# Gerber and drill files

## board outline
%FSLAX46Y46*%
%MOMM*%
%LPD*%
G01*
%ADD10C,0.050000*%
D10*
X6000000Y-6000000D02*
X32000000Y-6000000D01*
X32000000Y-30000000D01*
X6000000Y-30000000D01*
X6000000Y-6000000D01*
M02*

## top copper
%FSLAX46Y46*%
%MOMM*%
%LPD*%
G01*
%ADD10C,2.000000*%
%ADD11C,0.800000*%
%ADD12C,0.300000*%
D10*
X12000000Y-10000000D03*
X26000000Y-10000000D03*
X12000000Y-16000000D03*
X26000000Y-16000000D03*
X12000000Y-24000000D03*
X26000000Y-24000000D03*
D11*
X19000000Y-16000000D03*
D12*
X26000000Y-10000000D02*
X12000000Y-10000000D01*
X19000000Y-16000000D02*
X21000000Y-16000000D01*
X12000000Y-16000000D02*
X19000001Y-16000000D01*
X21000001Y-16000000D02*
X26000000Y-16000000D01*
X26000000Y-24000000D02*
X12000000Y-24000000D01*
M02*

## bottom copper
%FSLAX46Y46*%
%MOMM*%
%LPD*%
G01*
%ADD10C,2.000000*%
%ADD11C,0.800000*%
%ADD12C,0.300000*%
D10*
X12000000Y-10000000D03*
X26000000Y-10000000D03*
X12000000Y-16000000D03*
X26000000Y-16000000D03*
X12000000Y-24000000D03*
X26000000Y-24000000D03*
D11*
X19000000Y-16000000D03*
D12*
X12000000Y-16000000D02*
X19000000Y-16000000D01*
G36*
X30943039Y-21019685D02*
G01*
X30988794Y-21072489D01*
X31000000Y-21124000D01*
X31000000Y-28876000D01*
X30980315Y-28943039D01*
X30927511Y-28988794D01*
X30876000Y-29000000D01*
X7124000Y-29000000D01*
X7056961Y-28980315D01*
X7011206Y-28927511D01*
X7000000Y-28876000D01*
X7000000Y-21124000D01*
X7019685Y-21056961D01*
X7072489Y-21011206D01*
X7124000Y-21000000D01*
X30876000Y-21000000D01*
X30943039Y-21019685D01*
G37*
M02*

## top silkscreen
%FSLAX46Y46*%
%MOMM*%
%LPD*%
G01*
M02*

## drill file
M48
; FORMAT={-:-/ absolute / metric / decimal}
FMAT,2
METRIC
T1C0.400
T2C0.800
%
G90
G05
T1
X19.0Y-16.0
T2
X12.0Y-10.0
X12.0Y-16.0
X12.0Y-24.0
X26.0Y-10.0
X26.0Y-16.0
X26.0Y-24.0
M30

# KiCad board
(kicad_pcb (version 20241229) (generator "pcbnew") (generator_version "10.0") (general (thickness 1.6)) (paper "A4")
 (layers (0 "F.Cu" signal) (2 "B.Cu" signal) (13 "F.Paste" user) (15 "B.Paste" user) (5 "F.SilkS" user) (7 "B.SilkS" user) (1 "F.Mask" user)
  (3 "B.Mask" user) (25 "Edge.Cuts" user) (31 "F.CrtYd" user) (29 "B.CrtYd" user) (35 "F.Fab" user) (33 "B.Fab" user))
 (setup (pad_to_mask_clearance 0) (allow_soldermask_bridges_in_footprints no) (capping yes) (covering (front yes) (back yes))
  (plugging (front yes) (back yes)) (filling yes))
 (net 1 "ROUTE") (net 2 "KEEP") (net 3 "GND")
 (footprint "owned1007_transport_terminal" (layer "F.Cu") (at 12 10)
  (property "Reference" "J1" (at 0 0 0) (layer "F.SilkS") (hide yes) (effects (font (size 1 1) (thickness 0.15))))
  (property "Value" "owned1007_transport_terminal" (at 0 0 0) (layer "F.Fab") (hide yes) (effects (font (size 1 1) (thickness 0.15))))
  (pad "1" thru_hole circle (at 0 0) (size 2 2) (drill 0.8) (layers "*.Cu" "*.Mask") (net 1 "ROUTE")))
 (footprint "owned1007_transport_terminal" (layer "F.Cu") (at 26 10)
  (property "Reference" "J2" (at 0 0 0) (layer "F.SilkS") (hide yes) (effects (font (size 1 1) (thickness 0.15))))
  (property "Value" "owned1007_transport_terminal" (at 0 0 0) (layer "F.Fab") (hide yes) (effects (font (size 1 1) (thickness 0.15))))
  (pad "1" thru_hole circle (at 0 0) (size 2 2) (drill 0.8) (layers "*.Cu" "*.Mask") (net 1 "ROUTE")))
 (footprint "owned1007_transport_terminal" (layer "F.Cu") (at 12 16)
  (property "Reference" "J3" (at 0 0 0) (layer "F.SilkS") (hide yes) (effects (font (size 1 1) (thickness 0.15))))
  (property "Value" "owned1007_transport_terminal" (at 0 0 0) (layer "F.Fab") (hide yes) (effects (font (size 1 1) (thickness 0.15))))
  (pad "1" thru_hole circle (at 0 0) (size 2 2) (drill 0.8) (layers "*.Cu" "*.Mask") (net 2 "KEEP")))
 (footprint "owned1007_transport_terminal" (layer "F.Cu") (at 26 16)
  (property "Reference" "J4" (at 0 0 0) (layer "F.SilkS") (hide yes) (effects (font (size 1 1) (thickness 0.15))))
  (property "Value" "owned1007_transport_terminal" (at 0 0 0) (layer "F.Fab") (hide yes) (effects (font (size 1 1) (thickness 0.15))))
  (pad "1" thru_hole circle (at 0 0) (size 2 2) (drill 0.8) (layers "*.Cu" "*.Mask") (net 2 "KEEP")))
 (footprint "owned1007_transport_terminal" (layer "F.Cu") (at 12 24)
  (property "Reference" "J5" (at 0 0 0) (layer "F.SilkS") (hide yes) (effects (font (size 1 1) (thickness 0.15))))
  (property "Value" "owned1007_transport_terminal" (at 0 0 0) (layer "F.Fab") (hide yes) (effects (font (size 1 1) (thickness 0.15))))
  (pad "1" thru_hole circle (at 0 0) (size 2 2) (drill 0.8) (layers "*.Cu" "*.Mask") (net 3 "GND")))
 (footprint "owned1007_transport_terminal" (layer "F.Cu") (at 26 24)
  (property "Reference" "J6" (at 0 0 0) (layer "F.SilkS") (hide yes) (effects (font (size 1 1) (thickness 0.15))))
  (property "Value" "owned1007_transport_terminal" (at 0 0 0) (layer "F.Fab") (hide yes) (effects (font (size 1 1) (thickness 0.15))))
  (pad "1" thru_hole circle (at 0 0) (size 2 2) (drill 0.8) (layers "*.Cu" "*.Mask") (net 3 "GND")))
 (gr_rect (start 6 6) (end 32 30) (stroke (width 0.05) (type default)) (fill none) (layer "Edge.Cuts"))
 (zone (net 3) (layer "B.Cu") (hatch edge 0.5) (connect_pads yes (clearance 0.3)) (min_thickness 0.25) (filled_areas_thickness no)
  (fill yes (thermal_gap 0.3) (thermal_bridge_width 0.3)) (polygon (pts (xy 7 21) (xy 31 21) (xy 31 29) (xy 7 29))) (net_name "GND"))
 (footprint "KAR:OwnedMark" (layer "F.Cu") (at 10 28)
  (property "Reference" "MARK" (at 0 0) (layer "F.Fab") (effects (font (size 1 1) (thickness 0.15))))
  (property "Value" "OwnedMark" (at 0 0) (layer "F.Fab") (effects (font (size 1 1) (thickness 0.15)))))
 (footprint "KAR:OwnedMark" (layer "F.Cu") (at 13 28)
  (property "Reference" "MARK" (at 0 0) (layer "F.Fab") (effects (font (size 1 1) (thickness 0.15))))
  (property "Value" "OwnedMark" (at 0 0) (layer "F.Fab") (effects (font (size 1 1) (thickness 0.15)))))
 (segment (start 26 10) (end 12 10) (width 0.3) (layer "F.Cu") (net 1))
 (segment (start 19 16) (end 21 16) (width 0.3) (layer "F.Cu") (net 2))
 (segment (start 12 16) (end 19.000001 16) (width 0.3) (layer "F.Cu") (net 2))
 (segment (start 21.000001 16) (end 26 16) (width 0.3) (layer "F.Cu") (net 2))
 (via (at 19 16) (size 0.8) (drill 0.4) (layers "F.Cu" "B.Cu") (free yes) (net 2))
 (segment (start 12 16) (end 19 16) (width 0.3) (layer "B.Cu") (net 2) (locked yes))
 (segment (start 26 24) (end 12 24) (width 0.3) (layer "F.Cu") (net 3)))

